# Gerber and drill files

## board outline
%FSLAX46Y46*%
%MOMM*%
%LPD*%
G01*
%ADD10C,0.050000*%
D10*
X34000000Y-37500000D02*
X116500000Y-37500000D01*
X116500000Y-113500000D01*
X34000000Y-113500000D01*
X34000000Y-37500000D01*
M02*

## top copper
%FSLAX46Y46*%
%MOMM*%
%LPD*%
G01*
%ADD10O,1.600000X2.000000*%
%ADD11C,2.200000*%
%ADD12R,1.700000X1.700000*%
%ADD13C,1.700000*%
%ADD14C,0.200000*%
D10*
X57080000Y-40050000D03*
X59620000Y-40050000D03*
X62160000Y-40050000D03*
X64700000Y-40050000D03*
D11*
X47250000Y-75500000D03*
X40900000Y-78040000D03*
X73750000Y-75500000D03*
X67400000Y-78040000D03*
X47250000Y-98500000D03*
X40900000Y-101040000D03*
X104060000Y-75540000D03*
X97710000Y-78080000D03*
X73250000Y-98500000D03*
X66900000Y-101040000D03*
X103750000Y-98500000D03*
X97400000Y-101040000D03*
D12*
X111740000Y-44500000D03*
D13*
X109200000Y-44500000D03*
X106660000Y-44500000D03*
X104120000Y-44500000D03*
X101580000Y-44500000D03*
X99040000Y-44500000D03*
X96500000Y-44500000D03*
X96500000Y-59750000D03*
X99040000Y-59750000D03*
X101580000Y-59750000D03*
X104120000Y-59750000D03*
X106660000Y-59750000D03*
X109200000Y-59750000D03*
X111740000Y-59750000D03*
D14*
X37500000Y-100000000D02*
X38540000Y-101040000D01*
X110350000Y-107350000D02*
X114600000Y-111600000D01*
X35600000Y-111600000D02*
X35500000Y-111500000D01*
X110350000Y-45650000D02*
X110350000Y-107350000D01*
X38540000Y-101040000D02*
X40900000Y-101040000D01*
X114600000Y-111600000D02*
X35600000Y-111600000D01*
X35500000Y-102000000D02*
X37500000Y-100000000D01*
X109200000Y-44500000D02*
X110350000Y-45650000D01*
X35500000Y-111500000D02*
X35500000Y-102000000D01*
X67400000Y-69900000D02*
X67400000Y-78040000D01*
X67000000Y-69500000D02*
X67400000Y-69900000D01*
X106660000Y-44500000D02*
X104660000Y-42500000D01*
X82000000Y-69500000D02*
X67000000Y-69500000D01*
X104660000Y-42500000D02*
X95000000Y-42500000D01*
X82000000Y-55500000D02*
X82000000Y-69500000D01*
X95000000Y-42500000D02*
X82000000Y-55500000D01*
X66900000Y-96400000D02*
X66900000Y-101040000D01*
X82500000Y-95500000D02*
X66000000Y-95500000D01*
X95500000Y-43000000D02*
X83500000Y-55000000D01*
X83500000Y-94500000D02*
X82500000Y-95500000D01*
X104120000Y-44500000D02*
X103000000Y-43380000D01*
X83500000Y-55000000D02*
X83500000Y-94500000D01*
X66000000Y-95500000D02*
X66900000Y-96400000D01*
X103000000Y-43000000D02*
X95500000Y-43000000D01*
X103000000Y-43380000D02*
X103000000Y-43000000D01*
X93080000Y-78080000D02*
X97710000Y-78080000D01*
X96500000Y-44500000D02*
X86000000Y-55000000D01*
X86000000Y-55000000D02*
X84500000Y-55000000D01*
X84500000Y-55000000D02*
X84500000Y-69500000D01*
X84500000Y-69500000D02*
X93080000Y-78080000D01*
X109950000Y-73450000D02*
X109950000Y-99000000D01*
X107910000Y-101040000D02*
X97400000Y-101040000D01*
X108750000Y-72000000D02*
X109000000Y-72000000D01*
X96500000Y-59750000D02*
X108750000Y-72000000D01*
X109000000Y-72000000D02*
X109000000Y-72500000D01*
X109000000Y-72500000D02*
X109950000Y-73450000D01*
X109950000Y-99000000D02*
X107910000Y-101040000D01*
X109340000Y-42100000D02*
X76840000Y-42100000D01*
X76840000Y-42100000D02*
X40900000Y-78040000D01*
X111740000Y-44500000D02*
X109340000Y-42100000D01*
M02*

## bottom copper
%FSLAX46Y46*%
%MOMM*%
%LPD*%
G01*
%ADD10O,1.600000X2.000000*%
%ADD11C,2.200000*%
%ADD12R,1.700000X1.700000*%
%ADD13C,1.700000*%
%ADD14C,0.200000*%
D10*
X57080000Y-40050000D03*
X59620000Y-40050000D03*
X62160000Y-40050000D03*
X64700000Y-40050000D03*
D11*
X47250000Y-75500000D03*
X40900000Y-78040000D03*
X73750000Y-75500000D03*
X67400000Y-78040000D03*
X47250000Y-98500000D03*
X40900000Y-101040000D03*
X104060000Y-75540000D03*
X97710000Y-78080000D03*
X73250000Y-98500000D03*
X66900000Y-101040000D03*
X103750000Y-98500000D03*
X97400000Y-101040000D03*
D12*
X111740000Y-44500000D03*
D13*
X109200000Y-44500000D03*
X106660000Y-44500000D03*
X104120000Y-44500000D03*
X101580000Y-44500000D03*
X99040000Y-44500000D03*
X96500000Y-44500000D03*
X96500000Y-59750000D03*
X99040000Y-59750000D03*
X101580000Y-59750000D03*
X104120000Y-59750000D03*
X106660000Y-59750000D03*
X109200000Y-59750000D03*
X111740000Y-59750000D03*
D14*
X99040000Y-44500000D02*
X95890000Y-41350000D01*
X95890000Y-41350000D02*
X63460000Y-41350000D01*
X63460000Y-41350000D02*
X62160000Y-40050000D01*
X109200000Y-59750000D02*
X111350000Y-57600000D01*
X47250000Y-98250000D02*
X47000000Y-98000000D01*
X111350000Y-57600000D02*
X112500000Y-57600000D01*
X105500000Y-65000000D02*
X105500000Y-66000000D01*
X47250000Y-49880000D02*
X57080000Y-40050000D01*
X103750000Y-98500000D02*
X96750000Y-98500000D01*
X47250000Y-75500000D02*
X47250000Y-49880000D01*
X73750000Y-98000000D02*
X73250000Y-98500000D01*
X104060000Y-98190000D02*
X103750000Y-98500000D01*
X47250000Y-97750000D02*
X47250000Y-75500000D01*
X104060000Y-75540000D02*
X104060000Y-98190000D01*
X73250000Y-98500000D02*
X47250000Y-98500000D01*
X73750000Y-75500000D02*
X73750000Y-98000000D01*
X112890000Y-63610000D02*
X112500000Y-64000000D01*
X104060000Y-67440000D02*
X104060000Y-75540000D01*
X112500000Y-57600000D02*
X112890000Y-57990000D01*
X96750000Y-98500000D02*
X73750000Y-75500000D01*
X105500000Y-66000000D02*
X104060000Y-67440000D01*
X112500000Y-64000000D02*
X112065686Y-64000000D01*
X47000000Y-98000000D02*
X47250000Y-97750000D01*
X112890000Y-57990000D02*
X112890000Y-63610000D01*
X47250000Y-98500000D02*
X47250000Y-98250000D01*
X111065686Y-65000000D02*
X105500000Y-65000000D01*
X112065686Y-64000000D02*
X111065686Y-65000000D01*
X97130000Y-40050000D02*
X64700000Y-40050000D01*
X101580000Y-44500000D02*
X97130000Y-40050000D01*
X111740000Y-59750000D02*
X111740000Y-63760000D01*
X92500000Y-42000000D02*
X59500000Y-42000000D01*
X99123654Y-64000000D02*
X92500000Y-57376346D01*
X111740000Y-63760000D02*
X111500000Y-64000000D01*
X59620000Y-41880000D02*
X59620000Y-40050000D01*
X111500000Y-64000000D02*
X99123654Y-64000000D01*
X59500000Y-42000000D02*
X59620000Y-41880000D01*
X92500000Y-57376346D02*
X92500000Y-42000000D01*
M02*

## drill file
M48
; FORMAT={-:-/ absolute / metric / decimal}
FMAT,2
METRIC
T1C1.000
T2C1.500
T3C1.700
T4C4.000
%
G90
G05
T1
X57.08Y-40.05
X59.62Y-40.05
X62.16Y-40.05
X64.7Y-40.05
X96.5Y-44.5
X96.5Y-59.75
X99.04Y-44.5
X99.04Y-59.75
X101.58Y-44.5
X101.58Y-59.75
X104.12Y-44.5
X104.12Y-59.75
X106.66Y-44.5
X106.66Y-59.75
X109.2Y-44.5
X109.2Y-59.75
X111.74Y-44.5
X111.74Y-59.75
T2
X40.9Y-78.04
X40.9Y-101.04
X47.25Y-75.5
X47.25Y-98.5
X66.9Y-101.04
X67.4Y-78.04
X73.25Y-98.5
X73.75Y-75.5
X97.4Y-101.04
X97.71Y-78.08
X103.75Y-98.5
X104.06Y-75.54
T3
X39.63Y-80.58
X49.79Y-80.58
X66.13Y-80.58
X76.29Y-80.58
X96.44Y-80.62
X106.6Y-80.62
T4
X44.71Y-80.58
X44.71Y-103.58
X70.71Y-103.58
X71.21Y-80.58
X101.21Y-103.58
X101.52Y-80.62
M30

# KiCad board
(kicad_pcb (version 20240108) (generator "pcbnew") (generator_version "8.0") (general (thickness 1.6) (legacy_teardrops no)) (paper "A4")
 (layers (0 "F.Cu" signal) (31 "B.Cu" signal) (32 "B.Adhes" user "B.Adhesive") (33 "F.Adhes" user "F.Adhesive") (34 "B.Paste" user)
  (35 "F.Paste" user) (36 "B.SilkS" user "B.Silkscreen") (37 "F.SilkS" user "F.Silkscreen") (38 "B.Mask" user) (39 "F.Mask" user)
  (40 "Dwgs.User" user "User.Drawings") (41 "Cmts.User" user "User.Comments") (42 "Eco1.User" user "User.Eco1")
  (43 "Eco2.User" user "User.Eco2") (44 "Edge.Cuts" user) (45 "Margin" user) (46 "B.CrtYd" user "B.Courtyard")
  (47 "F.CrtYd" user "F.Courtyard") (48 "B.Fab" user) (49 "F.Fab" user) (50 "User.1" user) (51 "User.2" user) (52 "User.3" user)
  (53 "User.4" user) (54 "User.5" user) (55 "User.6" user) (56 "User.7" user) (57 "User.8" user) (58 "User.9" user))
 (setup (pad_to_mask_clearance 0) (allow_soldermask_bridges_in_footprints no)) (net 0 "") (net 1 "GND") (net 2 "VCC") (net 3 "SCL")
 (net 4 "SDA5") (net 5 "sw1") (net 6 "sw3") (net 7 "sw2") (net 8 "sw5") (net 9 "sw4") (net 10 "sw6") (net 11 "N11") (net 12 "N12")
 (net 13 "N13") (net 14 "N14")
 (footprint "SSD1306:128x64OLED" (layer "F.Cu") (at 60.7 50.65)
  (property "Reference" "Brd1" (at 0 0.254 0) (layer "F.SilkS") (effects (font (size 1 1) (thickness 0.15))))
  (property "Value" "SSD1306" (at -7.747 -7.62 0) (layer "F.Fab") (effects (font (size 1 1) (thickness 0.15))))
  (pad "1" thru_hole oval (at -3.62 -10.6 90) (size 2 1.6) (drill 1) (layers "*.Cu" "*.Mask") (remove_unused_layers no) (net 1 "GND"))
  (pad "2" thru_hole oval (at -1.08 -10.6 90) (size 2 1.6) (drill 1) (layers "*.Cu" "*.Mask") (remove_unused_layers no) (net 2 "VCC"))
  (pad "3" thru_hole oval (at 1.46 -10.6 90) (size 2 1.6) (drill 1) (layers "*.Cu" "*.Mask") (remove_unused_layers no) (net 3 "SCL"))
  (pad "4" thru_hole oval (at 4 -10.6 90) (size 2 1.6) (drill 1) (layers "*.Cu" "*.Mask") (remove_unused_layers no) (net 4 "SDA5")))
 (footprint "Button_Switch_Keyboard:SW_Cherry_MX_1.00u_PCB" (layer "F.Cu") (at 47.25 75.5)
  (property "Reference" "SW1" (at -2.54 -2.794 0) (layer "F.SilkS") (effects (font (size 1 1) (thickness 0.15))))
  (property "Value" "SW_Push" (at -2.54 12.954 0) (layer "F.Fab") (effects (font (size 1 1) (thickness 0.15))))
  (pad "" np_thru_hole circle (at -7.62 5.08) (size 1.7 1.7) (drill 1.7) (layers "*.Cu" "*.Mask"))
  (pad "" np_thru_hole circle (at -2.54 5.08) (size 4 4) (drill 4) (layers "*.Cu" "*.Mask"))
  (pad "" np_thru_hole circle (at 2.54 5.08) (size 1.7 1.7) (drill 1.7) (layers "*.Cu" "*.Mask"))
  (pad "1" thru_hole circle (at 0 0) (size 2.2 2.2) (drill 1.5) (layers "*.Cu" "*.Mask") (remove_unused_layers no) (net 1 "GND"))
  (pad "2" thru_hole circle (at -6.35 2.54) (size 2.2 2.2) (drill 1.5) (layers "*.Cu" "*.Mask") (remove_unused_layers no) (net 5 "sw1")))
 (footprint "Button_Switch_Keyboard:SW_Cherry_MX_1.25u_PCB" (layer "F.Cu") (at 73.75 75.5)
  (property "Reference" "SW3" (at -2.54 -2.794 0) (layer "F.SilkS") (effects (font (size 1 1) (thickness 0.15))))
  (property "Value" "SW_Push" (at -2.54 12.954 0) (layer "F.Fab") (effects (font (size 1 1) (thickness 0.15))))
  (pad "" np_thru_hole circle (at -7.62 5.08) (size 1.7 1.7) (drill 1.7) (layers "*.Cu" "*.Mask"))
  (pad "" np_thru_hole circle (at -2.54 5.08) (size 4 4) (drill 4) (layers "*.Cu" "*.Mask"))
  (pad "" np_thru_hole circle (at 2.54 5.08) (size 1.7 1.7) (drill 1.7) (layers "*.Cu" "*.Mask"))
  (pad "1" thru_hole circle (at 0 0) (size 2.2 2.2) (drill 1.5) (layers "*.Cu" "*.Mask") (remove_unused_layers no) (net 1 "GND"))
  (pad "2" thru_hole circle (at -6.35 2.54) (size 2.2 2.2) (drill 1.5) (layers "*.Cu" "*.Mask") (remove_unused_layers no) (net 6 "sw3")))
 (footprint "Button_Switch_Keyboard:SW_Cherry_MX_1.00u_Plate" (layer "F.Cu") (at 47.25 98.5)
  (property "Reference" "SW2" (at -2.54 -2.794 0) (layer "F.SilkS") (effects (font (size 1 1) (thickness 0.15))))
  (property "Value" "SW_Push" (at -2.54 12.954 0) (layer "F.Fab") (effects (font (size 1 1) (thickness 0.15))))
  (pad "" np_thru_hole circle (at -2.54 5.08) (size 4 4) (drill 4) (layers "*.Cu" "*.Mask"))
  (pad "1" thru_hole circle (at 0 0) (size 2.2 2.2) (drill 1.5) (layers "*.Cu" "*.Mask") (remove_unused_layers no) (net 1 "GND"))
  (pad "2" thru_hole circle (at -6.35 2.54) (size 2.2 2.2) (drill 1.5) (layers "*.Cu" "*.Mask") (remove_unused_layers no) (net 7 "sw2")))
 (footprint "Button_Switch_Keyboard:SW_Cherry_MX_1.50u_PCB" (layer "F.Cu") (at 104.06 75.54)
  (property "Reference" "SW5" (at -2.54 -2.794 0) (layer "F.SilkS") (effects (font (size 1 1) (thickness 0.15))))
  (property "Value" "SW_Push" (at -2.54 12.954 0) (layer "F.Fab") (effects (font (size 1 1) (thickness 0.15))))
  (pad "" np_thru_hole circle (at -7.62 5.08) (size 1.7 1.7) (drill 1.7) (layers "*.Cu" "*.Mask"))
  (pad "" np_thru_hole circle (at -2.54 5.08) (size 4 4) (drill 4) (layers "*.Cu" "*.Mask"))
  (pad "" np_thru_hole circle (at 2.54 5.08) (size 1.7 1.7) (drill 1.7) (layers "*.Cu" "*.Mask"))
  (pad "1" thru_hole circle (at 0 0) (size 2.2 2.2) (drill 1.5) (layers "*.Cu" "*.Mask") (remove_unused_layers no) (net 1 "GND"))
  (pad "2" thru_hole circle (at -6.35 2.54) (size 2.2 2.2) (drill 1.5) (layers "*.Cu" "*.Mask") (remove_unused_layers no) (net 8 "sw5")))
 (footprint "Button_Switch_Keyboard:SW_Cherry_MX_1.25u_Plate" (layer "F.Cu") (at 73.25 98.5)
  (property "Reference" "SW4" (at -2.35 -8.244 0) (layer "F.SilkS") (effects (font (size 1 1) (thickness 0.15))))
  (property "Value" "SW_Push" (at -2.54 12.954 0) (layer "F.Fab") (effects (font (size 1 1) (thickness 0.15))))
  (pad "" np_thru_hole circle (at -2.54 5.08) (size 4 4) (drill 4) (layers "*.Cu" "*.Mask"))
  (pad "1" thru_hole circle (at 0 0) (size 2.2 2.2) (drill 1.5) (layers "*.Cu" "*.Mask") (remove_unused_layers no) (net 1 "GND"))
  (pad "2" thru_hole circle (at -6.35 2.54) (size 2.2 2.2) (drill 1.5) (layers "*.Cu" "*.Mask") (remove_unused_layers no) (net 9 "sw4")))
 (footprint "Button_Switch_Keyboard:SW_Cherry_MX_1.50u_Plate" (layer "F.Cu") (at 103.75 98.5)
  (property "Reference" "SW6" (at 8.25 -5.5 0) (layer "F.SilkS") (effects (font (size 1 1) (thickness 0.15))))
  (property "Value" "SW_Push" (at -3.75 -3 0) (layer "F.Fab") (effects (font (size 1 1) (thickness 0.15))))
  (pad "" np_thru_hole circle (at -2.54 5.08) (size 4 4) (drill 4) (layers "*.Cu" "*.Mask"))
  (pad "1" thru_hole circle (at 0 0) (size 2.2 2.2) (drill 1.5) (layers "*.Cu" "*.Mask") (remove_unused_layers no) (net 1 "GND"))
  (pad "2" thru_hole circle (at -6.35 2.54) (size 2.2 2.2) (drill 1.5) (layers "*.Cu" "*.Mask") (remove_unused_layers no) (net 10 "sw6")))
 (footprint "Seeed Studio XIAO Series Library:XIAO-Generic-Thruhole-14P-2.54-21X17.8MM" (layer "F.Cu") (at 104.12 52.125 -90)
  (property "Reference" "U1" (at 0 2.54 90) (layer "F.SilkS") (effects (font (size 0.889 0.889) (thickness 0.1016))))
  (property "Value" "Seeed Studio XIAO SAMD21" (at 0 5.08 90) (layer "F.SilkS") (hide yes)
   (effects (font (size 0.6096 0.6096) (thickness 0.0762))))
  (pad "1" thru_hole rect (at -7.625 -7.62 270) (size 1.7 1.7) (drill 1) (layers "*.Cu" "*.Mask") (remove_unused_layers no) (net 5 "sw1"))
  (pad "2" thru_hole circle (at -7.625 -5.08 270) (size 1.7 1.7) (drill 1) (layers "*.Cu" "*.Mask") (remove_unused_layers no) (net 7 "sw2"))
  (pad "3" thru_hole circle (at -7.625 -2.54 270) (size 1.7 1.7) (drill 1) (layers "*.Cu" "*.Mask") (remove_unused_layers no) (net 6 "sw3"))
  (pad "4" thru_hole circle (at -7.625 0 270) (size 1.7 1.7) (drill 1) (layers "*.Cu" "*.Mask") (remove_unused_layers no) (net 9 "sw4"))
  (pad "5" thru_hole circle (at -7.625 2.54 270) (size 1.7 1.7) (drill 1) (layers "*.Cu" "*.Mask") (remove_unused_layers no) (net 4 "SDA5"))
  (pad "6" thru_hole circle (at -7.625 5.08 90) (size 1.7 1.7) (drill 1) (layers "*.Cu" "*.Mask") (remove_unused_layers no) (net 3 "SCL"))
  (pad "7" thru_hole circle (at -7.625 7.62 270) (size 1.7 1.7) (drill 1) (layers "*.Cu" "*.Mask") (remove_unused_layers no) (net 8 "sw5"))
  (pad "8" thru_hole circle (at 7.625 7.62 270) (size 1.7 1.7) (drill 1) (layers "*.Cu" "*.Mask") (remove_unused_layers no) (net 10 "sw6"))
  (pad "9" thru_hole circle (at 7.625 5.08 270) (size 1.7 1.7) (drill 1) (layers "*.Cu" "*.Mask") (remove_unused_layers no) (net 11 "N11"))
  (pad "10" thru_hole circle (at 7.625 2.54 270) (size 1.7 1.7) (drill 1) (layers "*.Cu" "*.Mask") (remove_unused_layers no) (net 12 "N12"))
  (pad "11" thru_hole circle (at 7.625 0 270) (size 1.7 1.7) (drill 1) (layers "*.Cu" "*.Mask") (remove_unused_layers no) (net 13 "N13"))
  (pad "12" thru_hole circle (at 7.625 -2.54 270) (size 1.7 1.7) (drill 1) (layers "*.Cu" "*.Mask") (remove_unused_layers no) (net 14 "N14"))
  (pad "13" thru_hole circle (at 7.625 -5.08 270) (size 1.7 1.7) (drill 1) (layers "*.Cu" "*.Mask") (remove_unused_layers no) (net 1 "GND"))
  (pad "14" thru_hole circle (at 7.625 -7.62 270) (size 1.7 1.7) (drill 1) (layers "*.Cu" "*.Mask") (remove_unused_layers no) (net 2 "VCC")))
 (gr_rect (start 34 37.5) (end 116.5 113.5) (stroke (width 0.05) (type default)) (fill none) (layer "Edge.Cuts"))
 (segment (start 99.04 44.5) (end 95.89 41.35) (width 0.2) (layer "B.Cu") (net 3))
 (segment (start 95.89 41.35) (end 63.46 41.35) (width 0.2) (layer "B.Cu") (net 3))
 (segment (start 63.46 41.35) (end 62.16 40.05) (width 0.2) (layer "B.Cu") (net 3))
 (segment (start 109.2 59.75) (end 111.35 57.6) (width 0.2) (layer "B.Cu") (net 1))
 (segment (start 47.25 98.25) (end 47 98) (width 0.2) (layer "B.Cu") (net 1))
 (segment (start 111.35 57.6) (end 112.5 57.6) (width 0.2) (layer "B.Cu") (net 1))
 (segment (start 105.5 65) (end 105.5 66) (width 0.2) (layer "B.Cu") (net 1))
 (segment (start 47.25 49.88) (end 57.08 40.05) (width 0.2) (layer "B.Cu") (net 1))
 (segment (start 103.75 98.5) (end 96.75 98.5) (width 0.2) (layer "B.Cu") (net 1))
 (segment (start 47.25 75.5) (end 47.25 49.88) (width 0.2) (layer "B.Cu") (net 1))
 (segment (start 73.75 98) (end 73.25 98.5) (width 0.2) (layer "B.Cu") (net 1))
 (segment (start 104.06 98.19) (end 103.75 98.5) (width 0.2) (layer "B.Cu") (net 1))
 (segment (start 47.25 97.75) (end 47.25 75.5) (width 0.2) (layer "B.Cu") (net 1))
 (segment (start 104.06 75.54) (end 104.06 98.19) (width 0.2) (layer "B.Cu") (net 1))
 (segment (start 73.25 98.5) (end 47.25 98.5) (width 0.2) (layer "B.Cu") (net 1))
 (segment (start 73.75 75.5) (end 73.75 98) (width 0.2) (layer "B.Cu") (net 1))
 (segment (start 112.89 63.61) (end 112.5 64) (width 0.2) (layer "B.Cu") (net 1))
 (segment (start 104.06 67.44) (end 104.06 75.54) (width 0.2) (layer "B.Cu") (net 1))
 (segment (start 112.5 57.6) (end 112.89 57.99) (width 0.2) (layer "B.Cu") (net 1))
 (segment (start 96.75 98.5) (end 73.75 75.5) (width 0.2) (layer "B.Cu") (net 1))
 (segment (start 105.5 66) (end 104.06 67.44) (width 0.2) (layer "B.Cu") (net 1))
 (segment (start 112.5 64) (end 112.065686 64) (width 0.2) (layer "B.Cu") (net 1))
 (segment (start 47 98) (end 47.25 97.75) (width 0.2) (layer "B.Cu") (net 1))
 (segment (start 112.89 57.99) (end 112.89 63.61) (width 0.2) (layer "B.Cu") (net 1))
 (segment (start 47.25 98.5) (end 47.25 98.25) (width 0.2) (layer "B.Cu") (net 1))
 (segment (start 111.065686 65) (end 105.5 65) (width 0.2) (layer "B.Cu") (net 1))
 (segment (start 112.065686 64) (end 111.065686 65) (width 0.2) (layer "B.Cu") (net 1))
 (segment (start 97.13 40.05) (end 64.7 40.05) (width 0.2) (layer "B.Cu") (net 4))
 (segment (start 101.58 44.5) (end 97.13 40.05) (width 0.2) (layer "B.Cu") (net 4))
 (segment (start 111.74 59.75) (end 111.74 63.76) (width 0.2) (layer "B.Cu") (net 2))
 (segment (start 92.5 42) (end 59.5 42) (width 0.2) (layer "B.Cu") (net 2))
 (segment (start 99.123654 64) (end 92.5 57.376346) (width 0.2) (layer "B.Cu") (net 2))
 (segment (start 111.74 63.76) (end 111.5 64) (width 0.2) (layer "B.Cu") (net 2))
 (segment (start 59.62 41.88) (end 59.62 40.05) (width 0.2) (layer "B.Cu") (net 2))
 (segment (start 111.5 64) (end 99.123654 64) (width 0.2) (layer "B.Cu") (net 2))
 (segment (start 59.5 42) (end 59.62 41.88) (width 0.2) (layer "B.Cu") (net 2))
 (segment (start 92.5 57.376346) (end 92.5 42) (width 0.2) (layer "B.Cu") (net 2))
 (segment (start 37.5 100) (end 38.54 101.04) (width 0.2) (layer "F.Cu") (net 7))
 (segment (start 110.35 107.35) (end 114.6 111.6) (width 0.2) (layer "F.Cu") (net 7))
 (segment (start 35.6 111.6) (end 35.5 111.5) (width 0.2) (layer "F.Cu") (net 7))
 (segment (start 110.35 45.65) (end 110.35 107.35) (width 0.2) (layer "F.Cu") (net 7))
 (segment (start 38.54 101.04) (end 40.9 101.04) (width 0.2) (layer "F.Cu") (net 7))
 (segment (start 114.6 111.6) (end 35.6 111.6) (width 0.2) (layer "F.Cu") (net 7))
 (segment (start 35.5 102) (end 37.5 100) (width 0.2) (layer "F.Cu") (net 7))
 (segment (start 109.2 44.5) (end 110.35 45.65) (width 0.2) (layer "F.Cu") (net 7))
 (segment (start 35.5 111.5) (end 35.5 102) (width 0.2) (layer "F.Cu") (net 7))
 (segment (start 67.4 69.9) (end 67.4 78.04) (width 0.2) (layer "F.Cu") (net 6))
 (segment (start 67 69.5) (end 67.4 69.9) (width 0.2) (layer "F.Cu") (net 6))
 (segment (start 106.66 44.5) (end 104.66 42.5) (width 0.2) (layer "F.Cu") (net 6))
 (segment (start 82 69.5) (end 67 69.5) (width 0.2) (layer "F.Cu") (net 6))
 (segment (start 104.66 42.5) (end 95 42.5) (width 0.2) (layer "F.Cu") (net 6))
 (segment (start 82 55.5) (end 82 69.5) (width 0.2) (layer "F.Cu") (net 6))
 (segment (start 95 42.5) (end 82 55.5) (width 0.2) (layer "F.Cu") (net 6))
 (segment (start 66.9 96.4) (end 66.9 101.04) (width 0.2) (layer "F.Cu") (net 9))
 (segment (start 82.5 95.5) (end 66 95.5) (width 0.2) (layer "F.Cu") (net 9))
 (segment (start 95.5 43) (end 83.5 55) (width 0.2) (layer "F.Cu") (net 9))
 (segment (start 83.5 94.5) (end 82.5 95.5) (width 0.2) (layer "F.Cu") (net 9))
 (segment (start 104.12 44.5) (end 103 43.38) (width 0.2) (layer "F.Cu") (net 9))
 (segment (start 83.5 55) (end 83.5 94.5) (width 0.2) (layer "F.Cu") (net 9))
 (segment (start 66 95.5) (end 66.9 96.4) (width 0.2) (layer "F.Cu") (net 9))
 (segment (start 103 43) (end 95.5 43) (width 0.2) (layer "F.Cu") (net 9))
 (segment (start 103 43.38) (end 103 43) (width 0.2) (layer "F.Cu") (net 9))
 (segment (start 93.08 78.08) (end 97.71 78.08) (width 0.2) (layer "F.Cu") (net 8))
 (segment (start 96.5 44.5) (end 86 55) (width 0.2) (layer "F.Cu") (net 8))
 (segment (start 86 55) (end 84.5 55) (width 0.2) (layer "F.Cu") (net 8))
 (segment (start 84.5 55) (end 84.5 69.5) (width 0.2) (layer "F.Cu") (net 8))
 (segment (start 84.5 69.5) (end 93.08 78.08) (width 0.2) (layer "F.Cu") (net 8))
 (segment (start 109.95 73.45) (end 109.95 99) (width 0.2) (layer "F.Cu") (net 10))
 (segment (start 107.91 101.04) (end 97.4 101.04) (width 0.2) (layer "F.Cu") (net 10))
 (segment (start 108.75 72) (end 109 72) (width 0.2) (layer "F.Cu") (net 10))
 (segment (start 96.5 59.75) (end 108.75 72) (width 0.2) (layer "F.Cu") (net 10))
 (segment (start 109 72) (end 109 72.5) (width 0.2) (layer "F.Cu") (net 10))
 (segment (start 109 72.5) (end 109.95 73.45) (width 0.2) (layer "F.Cu") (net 10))
 (segment (start 109.95 99) (end 107.91 101.04) (width 0.2) (layer "F.Cu") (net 10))
 (segment (start 109.34 42.1) (end 76.84 42.1) (width 0.2) (layer "F.Cu") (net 5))
 (segment (start 76.84 42.1) (end 40.9 78.04) (width 0.2) (layer "F.Cu") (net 5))
 (segment (start 111.74 44.5) (end 109.34 42.1) (width 0.2) (layer "F.Cu") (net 5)))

